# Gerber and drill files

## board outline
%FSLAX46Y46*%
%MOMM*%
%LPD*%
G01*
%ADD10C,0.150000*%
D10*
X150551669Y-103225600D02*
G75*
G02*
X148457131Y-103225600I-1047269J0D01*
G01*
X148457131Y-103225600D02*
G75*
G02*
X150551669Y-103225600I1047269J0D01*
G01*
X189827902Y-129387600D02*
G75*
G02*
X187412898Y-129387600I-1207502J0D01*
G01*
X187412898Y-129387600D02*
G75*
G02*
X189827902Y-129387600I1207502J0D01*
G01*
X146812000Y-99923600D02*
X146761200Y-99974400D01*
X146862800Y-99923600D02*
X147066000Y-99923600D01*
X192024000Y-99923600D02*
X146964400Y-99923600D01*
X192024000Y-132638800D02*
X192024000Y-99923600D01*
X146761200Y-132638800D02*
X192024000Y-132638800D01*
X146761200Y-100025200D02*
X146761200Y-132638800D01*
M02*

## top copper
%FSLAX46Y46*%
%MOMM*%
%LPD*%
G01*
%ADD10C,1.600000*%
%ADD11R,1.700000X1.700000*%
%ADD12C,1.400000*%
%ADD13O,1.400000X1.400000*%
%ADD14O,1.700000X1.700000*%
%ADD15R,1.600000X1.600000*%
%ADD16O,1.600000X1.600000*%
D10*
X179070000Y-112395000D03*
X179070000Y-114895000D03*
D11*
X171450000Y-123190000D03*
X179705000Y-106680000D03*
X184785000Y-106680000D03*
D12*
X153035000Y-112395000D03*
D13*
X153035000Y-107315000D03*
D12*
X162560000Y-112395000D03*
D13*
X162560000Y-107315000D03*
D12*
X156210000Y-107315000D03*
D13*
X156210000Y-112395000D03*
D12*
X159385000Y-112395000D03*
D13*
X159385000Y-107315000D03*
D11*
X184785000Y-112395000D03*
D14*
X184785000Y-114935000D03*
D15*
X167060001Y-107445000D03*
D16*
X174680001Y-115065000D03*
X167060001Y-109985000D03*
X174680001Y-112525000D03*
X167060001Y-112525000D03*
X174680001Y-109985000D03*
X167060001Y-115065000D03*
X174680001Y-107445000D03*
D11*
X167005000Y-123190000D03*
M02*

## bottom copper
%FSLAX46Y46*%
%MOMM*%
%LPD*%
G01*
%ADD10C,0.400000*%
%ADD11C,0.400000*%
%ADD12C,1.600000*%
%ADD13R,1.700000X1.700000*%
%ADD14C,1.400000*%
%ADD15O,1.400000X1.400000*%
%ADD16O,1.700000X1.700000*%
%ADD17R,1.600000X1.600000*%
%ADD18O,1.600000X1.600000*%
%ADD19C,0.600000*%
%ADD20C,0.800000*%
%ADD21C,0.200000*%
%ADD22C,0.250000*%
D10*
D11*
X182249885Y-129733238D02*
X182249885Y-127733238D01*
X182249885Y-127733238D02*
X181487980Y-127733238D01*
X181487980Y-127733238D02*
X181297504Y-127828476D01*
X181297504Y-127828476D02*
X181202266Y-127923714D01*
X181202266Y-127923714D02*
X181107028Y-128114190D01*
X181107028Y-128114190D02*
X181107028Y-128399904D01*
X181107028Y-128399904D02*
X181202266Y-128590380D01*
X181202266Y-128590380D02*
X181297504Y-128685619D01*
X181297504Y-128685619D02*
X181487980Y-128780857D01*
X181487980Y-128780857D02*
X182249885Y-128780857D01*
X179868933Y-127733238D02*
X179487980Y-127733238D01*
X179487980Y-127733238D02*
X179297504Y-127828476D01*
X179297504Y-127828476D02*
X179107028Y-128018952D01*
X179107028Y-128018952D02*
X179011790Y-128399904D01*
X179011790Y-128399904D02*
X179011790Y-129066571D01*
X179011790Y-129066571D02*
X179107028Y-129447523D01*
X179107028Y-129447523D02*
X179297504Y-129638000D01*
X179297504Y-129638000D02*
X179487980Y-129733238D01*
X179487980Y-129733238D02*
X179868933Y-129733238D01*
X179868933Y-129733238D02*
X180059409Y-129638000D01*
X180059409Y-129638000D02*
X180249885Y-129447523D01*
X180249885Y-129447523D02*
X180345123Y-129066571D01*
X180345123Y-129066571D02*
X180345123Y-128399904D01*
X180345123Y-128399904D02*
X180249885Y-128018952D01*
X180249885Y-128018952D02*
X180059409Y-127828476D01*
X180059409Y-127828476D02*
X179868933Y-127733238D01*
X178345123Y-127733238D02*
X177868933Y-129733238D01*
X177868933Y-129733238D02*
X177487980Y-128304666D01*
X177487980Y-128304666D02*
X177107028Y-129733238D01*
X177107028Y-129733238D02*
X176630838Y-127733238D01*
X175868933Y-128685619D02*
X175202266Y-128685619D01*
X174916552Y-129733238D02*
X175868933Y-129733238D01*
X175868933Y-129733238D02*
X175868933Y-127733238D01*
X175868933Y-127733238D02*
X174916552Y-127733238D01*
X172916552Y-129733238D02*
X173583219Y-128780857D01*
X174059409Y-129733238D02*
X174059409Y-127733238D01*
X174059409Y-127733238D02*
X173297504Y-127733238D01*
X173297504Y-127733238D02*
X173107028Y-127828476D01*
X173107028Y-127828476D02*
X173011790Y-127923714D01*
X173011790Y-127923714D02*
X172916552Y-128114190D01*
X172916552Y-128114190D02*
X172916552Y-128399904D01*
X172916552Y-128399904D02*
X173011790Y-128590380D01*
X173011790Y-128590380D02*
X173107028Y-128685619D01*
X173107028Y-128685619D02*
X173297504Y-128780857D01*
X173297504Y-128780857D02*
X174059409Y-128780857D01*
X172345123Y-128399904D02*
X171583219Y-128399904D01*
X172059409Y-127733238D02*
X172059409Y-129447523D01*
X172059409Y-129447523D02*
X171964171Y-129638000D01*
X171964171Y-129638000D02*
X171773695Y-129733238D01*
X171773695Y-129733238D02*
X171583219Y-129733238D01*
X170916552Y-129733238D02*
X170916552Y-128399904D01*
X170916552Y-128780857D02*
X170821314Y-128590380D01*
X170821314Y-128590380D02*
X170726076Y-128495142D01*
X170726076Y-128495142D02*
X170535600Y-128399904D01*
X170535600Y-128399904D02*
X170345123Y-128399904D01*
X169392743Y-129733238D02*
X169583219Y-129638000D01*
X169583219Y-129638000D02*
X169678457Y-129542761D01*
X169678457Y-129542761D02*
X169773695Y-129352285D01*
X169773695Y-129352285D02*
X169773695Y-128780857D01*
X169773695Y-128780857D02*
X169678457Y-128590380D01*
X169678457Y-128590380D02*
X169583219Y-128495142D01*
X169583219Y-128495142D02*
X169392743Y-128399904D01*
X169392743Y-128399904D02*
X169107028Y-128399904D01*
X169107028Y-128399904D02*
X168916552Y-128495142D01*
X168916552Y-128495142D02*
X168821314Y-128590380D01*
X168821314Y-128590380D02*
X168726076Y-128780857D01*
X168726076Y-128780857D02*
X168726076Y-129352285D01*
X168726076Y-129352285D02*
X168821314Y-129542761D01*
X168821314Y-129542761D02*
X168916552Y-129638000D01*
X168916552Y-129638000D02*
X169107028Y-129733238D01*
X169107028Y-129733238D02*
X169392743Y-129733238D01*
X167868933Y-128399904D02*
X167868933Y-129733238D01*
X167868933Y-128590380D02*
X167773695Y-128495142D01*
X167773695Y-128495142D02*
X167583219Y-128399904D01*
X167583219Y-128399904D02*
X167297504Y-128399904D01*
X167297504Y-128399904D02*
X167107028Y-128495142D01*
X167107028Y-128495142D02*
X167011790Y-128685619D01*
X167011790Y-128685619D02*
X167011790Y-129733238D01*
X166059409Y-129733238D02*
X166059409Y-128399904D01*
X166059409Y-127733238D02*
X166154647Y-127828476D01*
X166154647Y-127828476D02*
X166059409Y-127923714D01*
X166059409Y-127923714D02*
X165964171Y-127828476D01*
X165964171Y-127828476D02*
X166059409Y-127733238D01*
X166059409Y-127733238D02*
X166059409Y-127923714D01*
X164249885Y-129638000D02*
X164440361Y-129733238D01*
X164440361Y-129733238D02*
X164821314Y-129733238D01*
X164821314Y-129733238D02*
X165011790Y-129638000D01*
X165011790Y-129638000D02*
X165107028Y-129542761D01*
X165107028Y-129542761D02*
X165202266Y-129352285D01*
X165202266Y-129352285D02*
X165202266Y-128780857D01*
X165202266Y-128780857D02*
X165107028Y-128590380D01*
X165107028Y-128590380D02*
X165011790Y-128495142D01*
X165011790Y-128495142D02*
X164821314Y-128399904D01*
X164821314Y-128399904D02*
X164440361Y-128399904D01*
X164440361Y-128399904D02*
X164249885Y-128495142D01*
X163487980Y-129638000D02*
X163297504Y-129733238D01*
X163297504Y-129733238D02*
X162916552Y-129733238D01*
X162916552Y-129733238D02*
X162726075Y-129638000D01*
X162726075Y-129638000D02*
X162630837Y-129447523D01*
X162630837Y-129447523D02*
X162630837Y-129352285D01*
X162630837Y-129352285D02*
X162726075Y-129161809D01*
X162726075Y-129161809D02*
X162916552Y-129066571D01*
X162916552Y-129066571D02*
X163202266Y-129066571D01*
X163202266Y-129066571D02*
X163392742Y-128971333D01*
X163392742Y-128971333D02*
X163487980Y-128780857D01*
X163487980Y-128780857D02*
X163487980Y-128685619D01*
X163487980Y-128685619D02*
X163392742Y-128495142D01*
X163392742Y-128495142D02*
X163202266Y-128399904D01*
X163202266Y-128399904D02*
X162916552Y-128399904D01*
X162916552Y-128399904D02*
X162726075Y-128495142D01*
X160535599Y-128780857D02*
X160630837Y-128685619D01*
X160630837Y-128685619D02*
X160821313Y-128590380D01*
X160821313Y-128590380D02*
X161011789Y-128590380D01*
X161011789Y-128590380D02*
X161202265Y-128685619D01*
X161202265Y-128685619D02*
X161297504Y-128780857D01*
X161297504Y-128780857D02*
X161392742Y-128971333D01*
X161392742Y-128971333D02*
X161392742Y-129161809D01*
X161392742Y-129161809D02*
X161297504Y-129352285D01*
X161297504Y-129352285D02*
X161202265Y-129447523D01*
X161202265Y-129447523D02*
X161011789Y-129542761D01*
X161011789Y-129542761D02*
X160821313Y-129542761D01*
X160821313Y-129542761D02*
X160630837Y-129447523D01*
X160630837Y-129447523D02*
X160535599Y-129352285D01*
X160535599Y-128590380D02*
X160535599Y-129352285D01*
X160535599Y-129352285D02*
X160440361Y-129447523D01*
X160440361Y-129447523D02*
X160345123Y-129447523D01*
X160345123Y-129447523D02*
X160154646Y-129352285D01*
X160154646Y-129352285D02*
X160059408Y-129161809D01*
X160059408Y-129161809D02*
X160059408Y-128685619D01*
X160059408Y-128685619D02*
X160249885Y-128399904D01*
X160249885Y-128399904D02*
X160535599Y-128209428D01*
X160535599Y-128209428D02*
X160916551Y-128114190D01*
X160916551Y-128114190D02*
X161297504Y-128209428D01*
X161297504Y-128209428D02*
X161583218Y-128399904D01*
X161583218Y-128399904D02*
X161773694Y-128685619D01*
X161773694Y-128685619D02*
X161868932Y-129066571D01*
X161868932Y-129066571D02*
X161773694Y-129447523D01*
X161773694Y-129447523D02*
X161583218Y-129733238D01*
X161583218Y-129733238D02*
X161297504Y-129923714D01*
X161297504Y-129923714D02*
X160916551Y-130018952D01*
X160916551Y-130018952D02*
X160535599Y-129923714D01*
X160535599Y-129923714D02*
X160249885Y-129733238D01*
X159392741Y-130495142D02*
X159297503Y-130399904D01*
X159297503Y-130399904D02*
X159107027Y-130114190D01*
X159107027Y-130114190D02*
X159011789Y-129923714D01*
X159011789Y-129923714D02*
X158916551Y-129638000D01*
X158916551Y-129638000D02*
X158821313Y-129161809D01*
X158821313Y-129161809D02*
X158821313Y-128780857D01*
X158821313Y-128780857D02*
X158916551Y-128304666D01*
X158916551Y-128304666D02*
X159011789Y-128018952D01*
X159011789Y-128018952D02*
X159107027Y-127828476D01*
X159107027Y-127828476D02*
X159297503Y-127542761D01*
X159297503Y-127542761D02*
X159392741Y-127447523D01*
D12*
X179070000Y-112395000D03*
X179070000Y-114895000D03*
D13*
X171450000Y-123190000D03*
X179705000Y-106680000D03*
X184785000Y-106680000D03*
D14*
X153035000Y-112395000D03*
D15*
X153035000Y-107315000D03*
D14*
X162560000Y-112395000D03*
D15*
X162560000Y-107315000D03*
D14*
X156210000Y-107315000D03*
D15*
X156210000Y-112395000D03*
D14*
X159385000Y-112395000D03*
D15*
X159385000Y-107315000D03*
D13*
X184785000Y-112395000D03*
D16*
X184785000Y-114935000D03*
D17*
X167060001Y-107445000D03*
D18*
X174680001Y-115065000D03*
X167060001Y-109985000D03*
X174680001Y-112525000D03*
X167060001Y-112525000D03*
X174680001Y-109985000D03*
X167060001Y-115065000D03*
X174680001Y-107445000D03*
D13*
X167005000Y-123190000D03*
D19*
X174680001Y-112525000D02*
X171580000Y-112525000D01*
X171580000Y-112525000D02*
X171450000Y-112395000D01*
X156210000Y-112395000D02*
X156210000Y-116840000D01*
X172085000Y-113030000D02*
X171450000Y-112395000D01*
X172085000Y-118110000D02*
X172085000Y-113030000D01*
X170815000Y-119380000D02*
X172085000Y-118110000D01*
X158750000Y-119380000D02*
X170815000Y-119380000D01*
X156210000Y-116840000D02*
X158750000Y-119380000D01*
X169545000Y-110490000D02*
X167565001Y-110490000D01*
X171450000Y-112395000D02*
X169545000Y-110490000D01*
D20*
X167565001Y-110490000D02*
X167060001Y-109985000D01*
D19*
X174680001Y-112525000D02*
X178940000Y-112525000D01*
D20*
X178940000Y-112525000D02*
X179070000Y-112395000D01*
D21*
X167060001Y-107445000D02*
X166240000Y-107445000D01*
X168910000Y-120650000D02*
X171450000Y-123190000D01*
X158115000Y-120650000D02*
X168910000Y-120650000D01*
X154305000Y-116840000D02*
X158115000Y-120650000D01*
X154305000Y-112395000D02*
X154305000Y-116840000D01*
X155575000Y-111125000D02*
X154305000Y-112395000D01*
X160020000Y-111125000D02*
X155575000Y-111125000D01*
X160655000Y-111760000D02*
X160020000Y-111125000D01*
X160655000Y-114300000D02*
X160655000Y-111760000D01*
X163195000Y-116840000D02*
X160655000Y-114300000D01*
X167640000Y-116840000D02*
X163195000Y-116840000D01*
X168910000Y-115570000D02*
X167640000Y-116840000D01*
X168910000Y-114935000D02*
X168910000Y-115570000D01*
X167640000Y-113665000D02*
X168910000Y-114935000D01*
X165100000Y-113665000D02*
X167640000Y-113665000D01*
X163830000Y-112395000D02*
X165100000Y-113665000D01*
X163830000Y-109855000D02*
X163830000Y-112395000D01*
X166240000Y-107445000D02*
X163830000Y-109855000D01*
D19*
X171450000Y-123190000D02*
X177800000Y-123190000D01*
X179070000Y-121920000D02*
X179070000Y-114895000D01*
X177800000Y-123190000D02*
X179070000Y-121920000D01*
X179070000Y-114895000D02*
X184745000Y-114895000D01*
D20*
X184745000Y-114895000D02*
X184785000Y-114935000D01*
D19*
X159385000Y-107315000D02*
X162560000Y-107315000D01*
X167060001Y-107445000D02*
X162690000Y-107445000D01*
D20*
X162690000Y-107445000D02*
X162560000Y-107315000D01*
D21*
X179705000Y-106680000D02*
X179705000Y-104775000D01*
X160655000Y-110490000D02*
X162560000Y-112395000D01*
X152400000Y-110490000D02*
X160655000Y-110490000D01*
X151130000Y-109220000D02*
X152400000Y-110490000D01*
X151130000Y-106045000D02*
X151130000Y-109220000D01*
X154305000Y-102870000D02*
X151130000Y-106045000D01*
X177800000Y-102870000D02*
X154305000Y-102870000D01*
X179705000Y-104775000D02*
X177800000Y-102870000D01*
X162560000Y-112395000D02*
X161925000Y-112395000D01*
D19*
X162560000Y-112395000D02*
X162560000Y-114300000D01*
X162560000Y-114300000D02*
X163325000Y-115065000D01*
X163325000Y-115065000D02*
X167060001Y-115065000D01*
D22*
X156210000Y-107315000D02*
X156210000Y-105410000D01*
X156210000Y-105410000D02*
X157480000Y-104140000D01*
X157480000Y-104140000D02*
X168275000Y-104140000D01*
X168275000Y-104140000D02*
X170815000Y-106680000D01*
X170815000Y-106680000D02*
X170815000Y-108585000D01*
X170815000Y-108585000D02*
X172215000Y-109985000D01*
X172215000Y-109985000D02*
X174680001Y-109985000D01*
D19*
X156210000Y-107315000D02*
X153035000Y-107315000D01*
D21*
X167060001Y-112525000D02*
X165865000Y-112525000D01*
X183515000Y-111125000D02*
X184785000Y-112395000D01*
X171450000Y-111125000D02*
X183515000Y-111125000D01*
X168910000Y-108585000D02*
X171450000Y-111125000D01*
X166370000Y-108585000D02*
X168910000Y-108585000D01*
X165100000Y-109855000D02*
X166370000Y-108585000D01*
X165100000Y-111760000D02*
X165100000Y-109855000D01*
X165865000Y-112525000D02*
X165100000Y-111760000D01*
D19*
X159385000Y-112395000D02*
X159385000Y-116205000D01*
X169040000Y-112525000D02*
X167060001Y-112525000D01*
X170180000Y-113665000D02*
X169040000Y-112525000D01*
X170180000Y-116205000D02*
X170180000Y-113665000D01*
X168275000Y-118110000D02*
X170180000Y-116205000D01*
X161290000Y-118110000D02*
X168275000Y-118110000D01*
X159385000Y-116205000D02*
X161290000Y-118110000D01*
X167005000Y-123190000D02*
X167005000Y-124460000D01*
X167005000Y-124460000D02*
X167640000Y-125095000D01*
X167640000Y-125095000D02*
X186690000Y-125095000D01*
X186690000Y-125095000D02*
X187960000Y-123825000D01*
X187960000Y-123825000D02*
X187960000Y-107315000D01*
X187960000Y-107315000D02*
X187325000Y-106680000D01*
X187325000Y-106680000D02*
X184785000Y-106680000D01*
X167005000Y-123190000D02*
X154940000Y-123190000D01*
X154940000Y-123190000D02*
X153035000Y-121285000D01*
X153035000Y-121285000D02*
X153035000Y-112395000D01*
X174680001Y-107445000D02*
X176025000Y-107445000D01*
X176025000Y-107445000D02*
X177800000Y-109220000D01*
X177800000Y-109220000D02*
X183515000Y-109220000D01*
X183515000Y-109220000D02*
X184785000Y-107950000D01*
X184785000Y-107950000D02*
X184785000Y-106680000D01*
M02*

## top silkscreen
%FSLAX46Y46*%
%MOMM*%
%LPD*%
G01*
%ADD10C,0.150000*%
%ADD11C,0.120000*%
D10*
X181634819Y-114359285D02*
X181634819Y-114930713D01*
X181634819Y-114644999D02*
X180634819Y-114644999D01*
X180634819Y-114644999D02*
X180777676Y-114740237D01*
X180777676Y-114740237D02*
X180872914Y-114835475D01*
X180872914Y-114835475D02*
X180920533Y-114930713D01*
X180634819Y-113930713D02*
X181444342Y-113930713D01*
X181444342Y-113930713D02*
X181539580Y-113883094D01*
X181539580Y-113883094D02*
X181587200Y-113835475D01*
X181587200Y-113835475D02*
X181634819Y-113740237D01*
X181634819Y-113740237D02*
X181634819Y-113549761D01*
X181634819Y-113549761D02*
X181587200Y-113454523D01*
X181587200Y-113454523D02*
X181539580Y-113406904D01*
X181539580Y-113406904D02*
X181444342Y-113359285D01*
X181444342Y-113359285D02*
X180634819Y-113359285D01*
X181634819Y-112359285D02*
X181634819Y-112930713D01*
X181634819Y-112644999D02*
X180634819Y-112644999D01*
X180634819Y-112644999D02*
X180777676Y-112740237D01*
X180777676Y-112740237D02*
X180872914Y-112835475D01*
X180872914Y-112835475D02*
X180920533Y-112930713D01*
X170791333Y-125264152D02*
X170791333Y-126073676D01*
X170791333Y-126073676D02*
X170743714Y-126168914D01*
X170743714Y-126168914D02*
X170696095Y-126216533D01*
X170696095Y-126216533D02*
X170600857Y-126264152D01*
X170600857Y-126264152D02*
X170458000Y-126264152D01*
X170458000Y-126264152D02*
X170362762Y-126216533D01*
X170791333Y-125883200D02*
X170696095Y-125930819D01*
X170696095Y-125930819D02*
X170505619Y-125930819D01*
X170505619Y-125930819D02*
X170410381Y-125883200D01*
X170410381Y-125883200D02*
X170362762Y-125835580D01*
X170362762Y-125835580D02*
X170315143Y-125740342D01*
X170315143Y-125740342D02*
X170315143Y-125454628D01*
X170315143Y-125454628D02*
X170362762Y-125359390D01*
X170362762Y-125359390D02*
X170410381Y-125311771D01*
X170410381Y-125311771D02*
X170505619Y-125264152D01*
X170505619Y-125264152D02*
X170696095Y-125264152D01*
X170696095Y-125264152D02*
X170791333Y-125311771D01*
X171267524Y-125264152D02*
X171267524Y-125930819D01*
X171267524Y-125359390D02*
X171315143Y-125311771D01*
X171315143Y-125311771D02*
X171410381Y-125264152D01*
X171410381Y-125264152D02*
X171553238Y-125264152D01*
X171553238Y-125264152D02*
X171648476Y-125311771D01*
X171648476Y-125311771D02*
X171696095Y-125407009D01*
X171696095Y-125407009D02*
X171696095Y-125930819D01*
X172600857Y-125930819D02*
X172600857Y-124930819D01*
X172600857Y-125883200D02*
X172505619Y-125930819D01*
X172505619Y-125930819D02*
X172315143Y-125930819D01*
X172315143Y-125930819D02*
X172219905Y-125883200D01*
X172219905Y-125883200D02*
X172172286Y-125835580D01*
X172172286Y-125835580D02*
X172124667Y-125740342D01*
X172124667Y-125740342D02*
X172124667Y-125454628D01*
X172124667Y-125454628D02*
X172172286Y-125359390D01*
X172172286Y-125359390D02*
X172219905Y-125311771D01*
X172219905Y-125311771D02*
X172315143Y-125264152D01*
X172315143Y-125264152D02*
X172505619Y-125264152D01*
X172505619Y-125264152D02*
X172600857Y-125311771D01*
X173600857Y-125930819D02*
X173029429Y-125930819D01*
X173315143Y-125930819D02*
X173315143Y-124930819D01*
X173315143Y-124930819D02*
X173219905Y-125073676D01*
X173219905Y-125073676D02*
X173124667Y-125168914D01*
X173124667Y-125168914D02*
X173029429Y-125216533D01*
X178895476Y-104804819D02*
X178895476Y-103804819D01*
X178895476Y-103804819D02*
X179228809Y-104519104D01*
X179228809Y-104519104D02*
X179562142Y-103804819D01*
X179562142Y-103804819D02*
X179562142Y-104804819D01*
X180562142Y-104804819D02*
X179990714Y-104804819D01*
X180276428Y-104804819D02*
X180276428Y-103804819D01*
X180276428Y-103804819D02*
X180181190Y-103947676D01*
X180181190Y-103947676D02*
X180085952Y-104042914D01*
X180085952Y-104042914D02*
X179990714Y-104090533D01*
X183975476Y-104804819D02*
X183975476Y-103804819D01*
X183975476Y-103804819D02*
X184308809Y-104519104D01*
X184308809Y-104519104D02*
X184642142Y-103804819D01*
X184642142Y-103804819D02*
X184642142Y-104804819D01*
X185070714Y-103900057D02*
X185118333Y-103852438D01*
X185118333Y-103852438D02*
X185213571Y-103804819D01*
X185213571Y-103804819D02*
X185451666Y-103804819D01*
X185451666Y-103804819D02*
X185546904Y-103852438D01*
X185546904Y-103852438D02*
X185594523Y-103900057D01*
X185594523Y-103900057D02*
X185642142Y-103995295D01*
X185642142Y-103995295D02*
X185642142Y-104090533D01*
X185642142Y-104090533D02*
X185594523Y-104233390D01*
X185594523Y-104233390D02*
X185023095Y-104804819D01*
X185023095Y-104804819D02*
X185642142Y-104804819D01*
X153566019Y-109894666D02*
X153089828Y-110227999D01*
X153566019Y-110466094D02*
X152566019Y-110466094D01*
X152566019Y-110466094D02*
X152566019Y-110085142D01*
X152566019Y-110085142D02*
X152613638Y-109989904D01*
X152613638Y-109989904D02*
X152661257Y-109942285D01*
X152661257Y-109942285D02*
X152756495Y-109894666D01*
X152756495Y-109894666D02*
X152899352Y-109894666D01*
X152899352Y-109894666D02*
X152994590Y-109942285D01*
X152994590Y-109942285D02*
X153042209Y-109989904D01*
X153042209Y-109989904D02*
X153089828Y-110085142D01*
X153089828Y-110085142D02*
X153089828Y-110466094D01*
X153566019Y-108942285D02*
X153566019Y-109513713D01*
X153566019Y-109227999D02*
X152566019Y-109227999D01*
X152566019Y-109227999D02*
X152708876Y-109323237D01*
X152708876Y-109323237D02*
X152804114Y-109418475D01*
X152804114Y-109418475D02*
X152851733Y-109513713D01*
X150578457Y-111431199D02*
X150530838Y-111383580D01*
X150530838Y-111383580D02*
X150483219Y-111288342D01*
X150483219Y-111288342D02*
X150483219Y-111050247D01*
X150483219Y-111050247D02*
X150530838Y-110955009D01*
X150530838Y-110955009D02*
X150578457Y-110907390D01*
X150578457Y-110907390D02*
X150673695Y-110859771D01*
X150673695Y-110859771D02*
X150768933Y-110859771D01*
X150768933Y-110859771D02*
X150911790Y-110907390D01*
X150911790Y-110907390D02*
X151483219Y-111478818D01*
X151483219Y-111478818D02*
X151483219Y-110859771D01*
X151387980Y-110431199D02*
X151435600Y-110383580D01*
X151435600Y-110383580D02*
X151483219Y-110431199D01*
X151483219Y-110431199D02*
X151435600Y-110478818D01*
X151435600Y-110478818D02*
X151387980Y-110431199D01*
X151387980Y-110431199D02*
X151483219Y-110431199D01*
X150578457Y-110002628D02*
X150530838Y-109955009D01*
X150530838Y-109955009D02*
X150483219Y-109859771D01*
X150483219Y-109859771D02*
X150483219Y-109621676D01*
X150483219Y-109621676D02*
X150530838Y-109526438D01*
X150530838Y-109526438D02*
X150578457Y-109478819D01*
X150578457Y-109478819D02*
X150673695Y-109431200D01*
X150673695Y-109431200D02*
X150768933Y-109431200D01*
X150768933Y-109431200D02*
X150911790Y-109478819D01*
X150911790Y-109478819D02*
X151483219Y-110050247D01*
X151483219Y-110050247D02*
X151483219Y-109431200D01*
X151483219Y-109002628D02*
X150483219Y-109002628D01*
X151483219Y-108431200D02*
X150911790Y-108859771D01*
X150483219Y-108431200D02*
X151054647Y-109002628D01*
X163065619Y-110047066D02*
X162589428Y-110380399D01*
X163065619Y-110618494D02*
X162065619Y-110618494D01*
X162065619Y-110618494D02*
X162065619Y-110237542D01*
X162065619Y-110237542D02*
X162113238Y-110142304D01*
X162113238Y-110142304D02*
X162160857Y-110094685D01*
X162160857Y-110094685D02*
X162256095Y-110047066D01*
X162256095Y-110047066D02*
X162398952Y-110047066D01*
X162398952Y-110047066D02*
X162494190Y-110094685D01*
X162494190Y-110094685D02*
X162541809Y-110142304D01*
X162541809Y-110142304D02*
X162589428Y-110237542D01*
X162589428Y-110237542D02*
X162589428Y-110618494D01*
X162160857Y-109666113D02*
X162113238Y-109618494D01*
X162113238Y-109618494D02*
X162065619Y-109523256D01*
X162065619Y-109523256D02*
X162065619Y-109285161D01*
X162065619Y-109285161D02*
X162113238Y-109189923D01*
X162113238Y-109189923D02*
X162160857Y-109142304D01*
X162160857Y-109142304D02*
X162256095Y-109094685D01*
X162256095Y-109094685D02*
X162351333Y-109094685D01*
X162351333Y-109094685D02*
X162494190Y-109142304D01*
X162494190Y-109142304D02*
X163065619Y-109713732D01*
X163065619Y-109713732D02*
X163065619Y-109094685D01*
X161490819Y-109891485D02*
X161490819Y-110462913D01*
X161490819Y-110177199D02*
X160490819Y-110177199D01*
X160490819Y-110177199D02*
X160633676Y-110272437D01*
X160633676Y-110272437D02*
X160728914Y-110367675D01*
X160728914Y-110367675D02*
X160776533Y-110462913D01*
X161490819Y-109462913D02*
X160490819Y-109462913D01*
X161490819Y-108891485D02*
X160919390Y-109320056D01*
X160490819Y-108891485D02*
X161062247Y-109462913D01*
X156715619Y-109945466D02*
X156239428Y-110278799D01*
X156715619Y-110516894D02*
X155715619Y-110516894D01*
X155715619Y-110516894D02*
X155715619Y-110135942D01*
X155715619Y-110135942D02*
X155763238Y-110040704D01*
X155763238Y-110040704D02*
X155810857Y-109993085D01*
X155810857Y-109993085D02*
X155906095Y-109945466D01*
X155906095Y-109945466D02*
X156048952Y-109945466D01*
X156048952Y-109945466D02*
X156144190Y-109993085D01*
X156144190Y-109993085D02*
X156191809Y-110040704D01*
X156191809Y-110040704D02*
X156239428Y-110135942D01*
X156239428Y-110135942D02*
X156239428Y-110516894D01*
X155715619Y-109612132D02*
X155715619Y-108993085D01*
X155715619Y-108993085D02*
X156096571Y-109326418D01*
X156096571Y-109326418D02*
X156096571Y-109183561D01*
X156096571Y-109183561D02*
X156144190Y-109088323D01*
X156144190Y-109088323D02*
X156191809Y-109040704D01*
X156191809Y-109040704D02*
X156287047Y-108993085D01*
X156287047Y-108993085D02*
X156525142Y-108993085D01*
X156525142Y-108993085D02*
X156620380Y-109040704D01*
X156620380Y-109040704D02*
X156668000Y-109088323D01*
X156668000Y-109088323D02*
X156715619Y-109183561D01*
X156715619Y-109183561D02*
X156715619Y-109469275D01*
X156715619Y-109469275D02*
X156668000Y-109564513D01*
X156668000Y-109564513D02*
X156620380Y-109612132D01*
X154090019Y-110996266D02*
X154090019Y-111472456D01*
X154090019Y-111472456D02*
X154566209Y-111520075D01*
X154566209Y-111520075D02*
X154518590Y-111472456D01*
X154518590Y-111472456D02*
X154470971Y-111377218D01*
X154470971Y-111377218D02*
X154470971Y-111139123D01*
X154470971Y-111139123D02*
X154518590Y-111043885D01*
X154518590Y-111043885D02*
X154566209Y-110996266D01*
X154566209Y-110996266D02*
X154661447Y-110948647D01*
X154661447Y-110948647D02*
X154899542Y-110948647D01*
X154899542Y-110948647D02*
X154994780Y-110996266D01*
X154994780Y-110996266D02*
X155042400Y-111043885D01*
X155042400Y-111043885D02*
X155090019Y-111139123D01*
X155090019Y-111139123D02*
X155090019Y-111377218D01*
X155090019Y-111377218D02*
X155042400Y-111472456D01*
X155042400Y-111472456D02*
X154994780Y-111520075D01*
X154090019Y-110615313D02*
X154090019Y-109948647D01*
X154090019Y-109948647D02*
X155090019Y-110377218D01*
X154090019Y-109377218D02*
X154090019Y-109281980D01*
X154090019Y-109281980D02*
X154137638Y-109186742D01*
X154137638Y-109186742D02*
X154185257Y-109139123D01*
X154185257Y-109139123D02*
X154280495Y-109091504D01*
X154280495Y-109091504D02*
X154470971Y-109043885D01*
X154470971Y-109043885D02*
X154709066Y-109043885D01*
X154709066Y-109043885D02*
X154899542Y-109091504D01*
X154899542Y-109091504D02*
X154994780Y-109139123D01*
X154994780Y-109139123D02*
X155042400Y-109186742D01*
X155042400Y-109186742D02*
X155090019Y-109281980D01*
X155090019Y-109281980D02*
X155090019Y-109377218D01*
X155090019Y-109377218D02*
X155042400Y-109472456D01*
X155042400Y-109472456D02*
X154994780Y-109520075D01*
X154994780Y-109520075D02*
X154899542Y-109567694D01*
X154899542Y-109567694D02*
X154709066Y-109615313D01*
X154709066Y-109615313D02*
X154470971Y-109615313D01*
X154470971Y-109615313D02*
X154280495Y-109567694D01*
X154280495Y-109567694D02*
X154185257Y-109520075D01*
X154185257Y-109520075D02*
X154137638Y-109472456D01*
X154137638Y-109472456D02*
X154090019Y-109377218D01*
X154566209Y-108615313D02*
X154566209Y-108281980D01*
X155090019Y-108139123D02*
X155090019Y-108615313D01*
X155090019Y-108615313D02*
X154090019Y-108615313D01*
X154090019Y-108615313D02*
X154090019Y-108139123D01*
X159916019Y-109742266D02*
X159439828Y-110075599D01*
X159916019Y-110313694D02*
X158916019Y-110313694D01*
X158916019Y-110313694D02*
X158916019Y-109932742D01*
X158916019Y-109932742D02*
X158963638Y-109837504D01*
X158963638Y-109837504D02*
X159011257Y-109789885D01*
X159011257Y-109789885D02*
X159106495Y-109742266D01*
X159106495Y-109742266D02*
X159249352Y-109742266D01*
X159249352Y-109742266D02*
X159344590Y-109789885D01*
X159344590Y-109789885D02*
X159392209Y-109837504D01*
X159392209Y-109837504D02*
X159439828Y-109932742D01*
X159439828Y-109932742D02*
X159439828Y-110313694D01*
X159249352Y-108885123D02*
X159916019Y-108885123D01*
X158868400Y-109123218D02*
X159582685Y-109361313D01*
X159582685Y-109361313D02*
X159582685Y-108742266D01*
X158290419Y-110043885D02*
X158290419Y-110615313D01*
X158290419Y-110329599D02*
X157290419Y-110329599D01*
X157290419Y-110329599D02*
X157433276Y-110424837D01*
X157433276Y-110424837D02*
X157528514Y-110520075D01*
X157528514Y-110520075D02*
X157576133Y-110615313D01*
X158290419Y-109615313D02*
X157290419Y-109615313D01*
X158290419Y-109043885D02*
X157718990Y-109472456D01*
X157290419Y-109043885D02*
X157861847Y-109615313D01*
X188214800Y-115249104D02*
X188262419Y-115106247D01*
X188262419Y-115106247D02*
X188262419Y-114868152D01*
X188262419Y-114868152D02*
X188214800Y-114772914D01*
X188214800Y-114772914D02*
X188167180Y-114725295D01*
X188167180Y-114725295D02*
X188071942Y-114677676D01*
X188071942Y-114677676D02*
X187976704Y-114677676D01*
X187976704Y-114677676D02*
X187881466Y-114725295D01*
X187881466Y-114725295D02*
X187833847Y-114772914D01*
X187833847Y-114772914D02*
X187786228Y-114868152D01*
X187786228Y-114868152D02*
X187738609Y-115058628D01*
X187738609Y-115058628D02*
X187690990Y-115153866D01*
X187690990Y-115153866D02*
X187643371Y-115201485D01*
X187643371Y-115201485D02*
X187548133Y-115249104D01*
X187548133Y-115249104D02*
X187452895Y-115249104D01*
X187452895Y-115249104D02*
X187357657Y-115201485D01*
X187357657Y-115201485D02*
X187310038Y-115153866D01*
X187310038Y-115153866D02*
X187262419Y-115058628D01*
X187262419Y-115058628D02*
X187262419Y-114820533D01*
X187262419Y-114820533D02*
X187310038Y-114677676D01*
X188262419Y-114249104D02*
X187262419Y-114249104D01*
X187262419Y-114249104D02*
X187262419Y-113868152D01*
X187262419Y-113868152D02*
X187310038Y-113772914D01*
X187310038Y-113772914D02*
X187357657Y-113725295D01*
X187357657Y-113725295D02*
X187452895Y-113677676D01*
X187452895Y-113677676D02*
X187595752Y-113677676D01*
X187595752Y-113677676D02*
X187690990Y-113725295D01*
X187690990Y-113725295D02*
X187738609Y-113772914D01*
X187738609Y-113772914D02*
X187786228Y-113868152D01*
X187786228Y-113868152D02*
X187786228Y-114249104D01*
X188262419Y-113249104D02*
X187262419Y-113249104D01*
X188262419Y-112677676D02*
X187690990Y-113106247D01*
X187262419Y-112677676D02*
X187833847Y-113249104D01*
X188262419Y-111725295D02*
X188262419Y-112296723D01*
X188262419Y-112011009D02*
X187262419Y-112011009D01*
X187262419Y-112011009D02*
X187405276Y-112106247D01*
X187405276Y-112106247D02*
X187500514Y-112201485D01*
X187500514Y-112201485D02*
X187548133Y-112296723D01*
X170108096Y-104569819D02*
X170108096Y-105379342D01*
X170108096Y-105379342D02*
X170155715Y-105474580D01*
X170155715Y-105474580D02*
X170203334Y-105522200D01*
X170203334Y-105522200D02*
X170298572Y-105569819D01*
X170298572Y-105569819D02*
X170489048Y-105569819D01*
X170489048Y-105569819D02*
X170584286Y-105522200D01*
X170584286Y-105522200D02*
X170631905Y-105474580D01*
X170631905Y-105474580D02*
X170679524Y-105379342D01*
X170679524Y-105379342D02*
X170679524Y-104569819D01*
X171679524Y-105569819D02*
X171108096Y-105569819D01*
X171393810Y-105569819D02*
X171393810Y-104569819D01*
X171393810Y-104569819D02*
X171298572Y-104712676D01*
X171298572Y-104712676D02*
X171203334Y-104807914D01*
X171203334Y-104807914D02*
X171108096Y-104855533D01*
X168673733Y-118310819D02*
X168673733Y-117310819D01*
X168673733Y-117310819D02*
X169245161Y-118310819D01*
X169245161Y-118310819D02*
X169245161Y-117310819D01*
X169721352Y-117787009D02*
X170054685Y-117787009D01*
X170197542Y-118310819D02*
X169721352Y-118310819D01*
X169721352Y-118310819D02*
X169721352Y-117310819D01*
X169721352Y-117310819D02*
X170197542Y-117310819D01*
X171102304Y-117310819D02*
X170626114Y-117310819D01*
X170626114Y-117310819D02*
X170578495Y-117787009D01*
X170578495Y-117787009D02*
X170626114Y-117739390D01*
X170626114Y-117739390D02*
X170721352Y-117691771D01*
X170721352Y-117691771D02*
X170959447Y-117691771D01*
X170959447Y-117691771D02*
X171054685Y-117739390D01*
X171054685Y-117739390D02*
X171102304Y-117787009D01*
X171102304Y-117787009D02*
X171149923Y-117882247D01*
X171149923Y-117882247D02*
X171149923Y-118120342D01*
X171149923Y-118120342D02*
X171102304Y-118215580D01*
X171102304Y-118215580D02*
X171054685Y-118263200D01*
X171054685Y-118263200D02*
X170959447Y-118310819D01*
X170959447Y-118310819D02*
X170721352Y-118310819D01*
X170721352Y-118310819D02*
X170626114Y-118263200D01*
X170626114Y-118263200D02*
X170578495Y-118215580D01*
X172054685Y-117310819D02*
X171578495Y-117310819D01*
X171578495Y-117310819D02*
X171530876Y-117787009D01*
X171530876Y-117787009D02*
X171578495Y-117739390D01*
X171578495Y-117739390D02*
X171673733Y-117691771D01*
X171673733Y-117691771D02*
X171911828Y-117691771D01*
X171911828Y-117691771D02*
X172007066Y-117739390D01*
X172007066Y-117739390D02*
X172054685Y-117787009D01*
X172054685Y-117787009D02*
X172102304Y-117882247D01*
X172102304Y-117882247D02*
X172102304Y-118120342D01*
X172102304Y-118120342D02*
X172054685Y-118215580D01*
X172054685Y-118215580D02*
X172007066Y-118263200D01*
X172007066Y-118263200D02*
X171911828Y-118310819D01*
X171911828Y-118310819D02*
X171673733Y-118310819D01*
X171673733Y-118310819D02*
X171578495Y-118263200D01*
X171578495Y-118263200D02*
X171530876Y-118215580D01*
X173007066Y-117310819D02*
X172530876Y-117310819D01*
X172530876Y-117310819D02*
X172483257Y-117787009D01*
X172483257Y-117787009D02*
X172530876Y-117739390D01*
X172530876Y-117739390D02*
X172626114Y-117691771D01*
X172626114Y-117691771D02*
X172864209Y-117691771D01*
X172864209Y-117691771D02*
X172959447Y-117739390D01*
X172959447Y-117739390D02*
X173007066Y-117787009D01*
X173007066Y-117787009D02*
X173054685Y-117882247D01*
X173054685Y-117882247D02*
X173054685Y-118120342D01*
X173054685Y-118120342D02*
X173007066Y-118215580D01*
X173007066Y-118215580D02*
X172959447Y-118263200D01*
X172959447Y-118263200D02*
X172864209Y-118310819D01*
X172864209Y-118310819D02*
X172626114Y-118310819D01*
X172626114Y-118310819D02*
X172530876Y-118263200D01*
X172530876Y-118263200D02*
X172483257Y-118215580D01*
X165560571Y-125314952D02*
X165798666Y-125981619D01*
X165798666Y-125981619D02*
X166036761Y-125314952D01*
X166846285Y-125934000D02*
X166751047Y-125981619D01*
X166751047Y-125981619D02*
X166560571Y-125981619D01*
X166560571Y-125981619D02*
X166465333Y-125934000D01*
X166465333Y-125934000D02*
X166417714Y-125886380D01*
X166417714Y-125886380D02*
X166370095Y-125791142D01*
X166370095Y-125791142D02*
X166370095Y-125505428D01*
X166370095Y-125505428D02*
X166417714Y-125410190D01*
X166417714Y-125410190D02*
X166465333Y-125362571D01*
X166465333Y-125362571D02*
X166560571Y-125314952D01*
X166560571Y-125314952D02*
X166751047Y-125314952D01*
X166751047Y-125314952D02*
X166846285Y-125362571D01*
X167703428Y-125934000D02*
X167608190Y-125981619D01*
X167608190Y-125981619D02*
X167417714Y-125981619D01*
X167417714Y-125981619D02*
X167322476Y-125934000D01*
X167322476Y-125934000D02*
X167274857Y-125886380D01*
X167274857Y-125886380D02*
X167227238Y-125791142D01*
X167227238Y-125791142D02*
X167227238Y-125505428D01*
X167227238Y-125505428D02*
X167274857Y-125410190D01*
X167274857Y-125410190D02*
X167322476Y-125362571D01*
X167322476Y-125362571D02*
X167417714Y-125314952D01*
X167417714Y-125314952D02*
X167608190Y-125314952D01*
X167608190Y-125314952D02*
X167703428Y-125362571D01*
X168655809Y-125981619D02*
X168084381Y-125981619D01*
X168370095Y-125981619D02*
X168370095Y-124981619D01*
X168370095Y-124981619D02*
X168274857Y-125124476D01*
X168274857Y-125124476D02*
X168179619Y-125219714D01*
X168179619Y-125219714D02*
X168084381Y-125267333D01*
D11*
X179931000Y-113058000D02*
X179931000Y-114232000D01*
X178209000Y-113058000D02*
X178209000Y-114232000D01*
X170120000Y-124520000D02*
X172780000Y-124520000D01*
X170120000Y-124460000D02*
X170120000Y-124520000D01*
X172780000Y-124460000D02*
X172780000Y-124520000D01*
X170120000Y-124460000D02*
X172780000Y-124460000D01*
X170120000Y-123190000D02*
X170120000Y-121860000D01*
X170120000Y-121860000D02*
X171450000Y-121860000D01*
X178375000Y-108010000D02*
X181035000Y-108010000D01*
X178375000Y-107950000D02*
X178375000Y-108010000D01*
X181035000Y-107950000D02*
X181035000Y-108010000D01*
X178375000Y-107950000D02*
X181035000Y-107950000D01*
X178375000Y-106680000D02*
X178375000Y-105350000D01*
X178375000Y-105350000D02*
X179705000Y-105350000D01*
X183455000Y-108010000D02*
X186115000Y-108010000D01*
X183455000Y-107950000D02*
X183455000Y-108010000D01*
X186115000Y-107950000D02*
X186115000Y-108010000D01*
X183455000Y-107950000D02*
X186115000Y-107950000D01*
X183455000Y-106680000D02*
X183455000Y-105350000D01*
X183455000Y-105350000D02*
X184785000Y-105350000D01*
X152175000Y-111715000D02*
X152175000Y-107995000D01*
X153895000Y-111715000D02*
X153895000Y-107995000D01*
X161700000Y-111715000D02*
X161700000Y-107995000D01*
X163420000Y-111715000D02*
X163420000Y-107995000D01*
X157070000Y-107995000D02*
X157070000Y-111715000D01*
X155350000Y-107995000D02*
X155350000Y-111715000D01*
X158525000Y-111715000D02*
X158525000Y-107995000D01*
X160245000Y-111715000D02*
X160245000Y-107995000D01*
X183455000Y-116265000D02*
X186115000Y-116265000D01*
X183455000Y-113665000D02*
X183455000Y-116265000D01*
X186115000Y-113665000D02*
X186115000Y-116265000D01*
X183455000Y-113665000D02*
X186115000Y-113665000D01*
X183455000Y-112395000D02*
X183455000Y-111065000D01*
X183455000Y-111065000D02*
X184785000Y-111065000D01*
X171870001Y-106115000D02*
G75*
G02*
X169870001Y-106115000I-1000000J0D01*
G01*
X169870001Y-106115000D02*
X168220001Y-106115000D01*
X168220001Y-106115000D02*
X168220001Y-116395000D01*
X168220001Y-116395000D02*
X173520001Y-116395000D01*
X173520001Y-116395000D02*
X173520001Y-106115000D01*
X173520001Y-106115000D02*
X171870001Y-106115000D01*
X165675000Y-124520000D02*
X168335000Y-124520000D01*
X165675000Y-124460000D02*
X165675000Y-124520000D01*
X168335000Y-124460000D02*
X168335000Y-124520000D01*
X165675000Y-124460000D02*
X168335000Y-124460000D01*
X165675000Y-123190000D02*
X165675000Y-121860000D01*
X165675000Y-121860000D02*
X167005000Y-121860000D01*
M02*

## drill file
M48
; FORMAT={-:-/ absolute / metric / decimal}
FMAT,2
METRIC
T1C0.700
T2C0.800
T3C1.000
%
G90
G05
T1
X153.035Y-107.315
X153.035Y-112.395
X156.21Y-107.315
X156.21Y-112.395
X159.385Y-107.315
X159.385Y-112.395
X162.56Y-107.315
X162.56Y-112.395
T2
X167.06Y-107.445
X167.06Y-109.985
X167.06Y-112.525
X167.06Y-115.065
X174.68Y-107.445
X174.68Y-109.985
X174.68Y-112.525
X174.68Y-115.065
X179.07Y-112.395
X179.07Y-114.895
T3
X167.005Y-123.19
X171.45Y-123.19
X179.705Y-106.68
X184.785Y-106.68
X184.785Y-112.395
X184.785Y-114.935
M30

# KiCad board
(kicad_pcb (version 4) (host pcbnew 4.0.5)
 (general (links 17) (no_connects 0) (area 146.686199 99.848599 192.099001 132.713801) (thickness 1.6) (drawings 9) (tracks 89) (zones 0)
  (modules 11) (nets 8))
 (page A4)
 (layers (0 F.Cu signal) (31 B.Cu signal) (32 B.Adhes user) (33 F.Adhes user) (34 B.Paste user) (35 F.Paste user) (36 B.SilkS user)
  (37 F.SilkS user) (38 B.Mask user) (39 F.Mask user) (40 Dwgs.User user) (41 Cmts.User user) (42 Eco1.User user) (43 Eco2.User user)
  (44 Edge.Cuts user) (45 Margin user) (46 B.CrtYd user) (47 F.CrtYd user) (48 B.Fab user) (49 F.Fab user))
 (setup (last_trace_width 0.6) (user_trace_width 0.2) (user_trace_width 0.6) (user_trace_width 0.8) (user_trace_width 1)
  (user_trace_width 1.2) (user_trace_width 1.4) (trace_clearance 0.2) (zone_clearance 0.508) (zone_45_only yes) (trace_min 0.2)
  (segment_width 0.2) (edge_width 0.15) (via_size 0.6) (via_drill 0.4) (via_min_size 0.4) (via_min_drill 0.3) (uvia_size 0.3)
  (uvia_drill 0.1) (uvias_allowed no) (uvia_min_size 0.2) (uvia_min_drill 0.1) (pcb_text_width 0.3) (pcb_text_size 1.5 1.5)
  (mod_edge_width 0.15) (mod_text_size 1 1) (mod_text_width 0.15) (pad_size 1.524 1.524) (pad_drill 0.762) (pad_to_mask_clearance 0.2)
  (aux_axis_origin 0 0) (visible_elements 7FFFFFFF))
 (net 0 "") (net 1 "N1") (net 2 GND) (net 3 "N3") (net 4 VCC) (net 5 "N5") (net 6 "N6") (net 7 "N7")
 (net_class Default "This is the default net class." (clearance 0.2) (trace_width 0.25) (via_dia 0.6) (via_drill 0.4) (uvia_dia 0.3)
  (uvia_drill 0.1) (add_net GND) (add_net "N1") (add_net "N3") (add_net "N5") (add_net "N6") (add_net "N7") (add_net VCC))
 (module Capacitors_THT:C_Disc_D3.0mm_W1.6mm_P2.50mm (layer F.Cu) (at 179.07 112.395 270)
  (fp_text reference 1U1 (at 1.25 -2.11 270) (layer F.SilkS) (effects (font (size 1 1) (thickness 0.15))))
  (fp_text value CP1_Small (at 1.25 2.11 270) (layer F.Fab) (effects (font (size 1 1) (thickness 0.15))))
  (fp_line (start 0.663 -0.861) (end 1.837 -0.861) (layer F.SilkS) (width 0.12))
  (fp_line (start 0.663 0.861) (end 1.837 0.861) (layer F.SilkS) (width 0.12))
  (pad 1 thru_hole circle (at 0 0 270) (size 1.6 1.6) (drill 0.8) (layers *.Cu *.Mask) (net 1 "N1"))
  (pad 2 thru_hole circle (at 2.5 0 270) (size 1.6 1.6) (drill 0.8) (layers *.Cu *.Mask) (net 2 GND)))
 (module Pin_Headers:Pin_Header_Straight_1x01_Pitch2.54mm (layer F.Cu) (at 171.45 123.19)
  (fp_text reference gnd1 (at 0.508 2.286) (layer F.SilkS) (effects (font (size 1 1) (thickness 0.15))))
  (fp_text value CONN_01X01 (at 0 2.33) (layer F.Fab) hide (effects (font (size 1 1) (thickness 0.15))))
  (fp_line (start -1.33 1.33) (end 1.33 1.33) (layer F.SilkS) (width 0.12))
  (fp_line (start -1.33 1.27) (end -1.33 1.33) (layer F.SilkS) (width 0.12))
  (fp_line (start 1.33 1.27) (end 1.33 1.33) (layer F.SilkS) (width 0.12))
  (fp_line (start -1.33 1.27) (end 1.33 1.27) (layer F.SilkS) (width 0.12))
  (fp_line (start -1.33 0) (end -1.33 -1.33) (layer F.SilkS) (width 0.12))
  (fp_line (start -1.33 -1.33) (end 0 -1.33) (layer F.SilkS) (width 0.12))
  (pad 1 thru_hole rect (at 0 0) (size 1.7 1.7) (drill 1) (layers *.Cu *.Mask) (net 2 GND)))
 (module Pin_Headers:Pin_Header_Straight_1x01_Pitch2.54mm (layer F.Cu) (at 179.705 106.68)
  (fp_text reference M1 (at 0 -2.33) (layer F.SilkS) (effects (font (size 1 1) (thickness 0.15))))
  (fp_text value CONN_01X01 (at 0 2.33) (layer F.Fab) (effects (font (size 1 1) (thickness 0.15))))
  (fp_line (start -1.33 1.33) (end 1.33 1.33) (layer F.SilkS) (width 0.12))
  (fp_line (start -1.33 1.27) (end -1.33 1.33) (layer F.SilkS) (width 0.12))
  (fp_line (start 1.33 1.27) (end 1.33 1.33) (layer F.SilkS) (width 0.12))
  (fp_line (start -1.33 1.27) (end 1.33 1.27) (layer F.SilkS) (width 0.12))
  (fp_line (start -1.33 0) (end -1.33 -1.33) (layer F.SilkS) (width 0.12))
  (fp_line (start -1.33 -1.33) (end 0 -1.33) (layer F.SilkS) (width 0.12))
  (pad 1 thru_hole rect (at 0 0) (size 1.7 1.7) (drill 1) (layers *.Cu *.Mask) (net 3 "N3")))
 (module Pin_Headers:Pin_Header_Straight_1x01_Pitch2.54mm (layer F.Cu) (at 184.785 106.68)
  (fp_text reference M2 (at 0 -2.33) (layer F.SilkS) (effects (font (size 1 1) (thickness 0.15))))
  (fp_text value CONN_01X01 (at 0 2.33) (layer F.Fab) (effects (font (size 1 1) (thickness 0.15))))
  (fp_line (start -1.33 1.33) (end 1.33 1.33) (layer F.SilkS) (width 0.12))
  (fp_line (start -1.33 1.27) (end -1.33 1.33) (layer F.SilkS) (width 0.12))
  (fp_line (start 1.33 1.27) (end 1.33 1.33) (layer F.SilkS) (width 0.12))
  (fp_line (start -1.33 1.27) (end 1.33 1.27) (layer F.SilkS) (width 0.12))
  (fp_line (start -1.33 0) (end -1.33 -1.33) (layer F.SilkS) (width 0.12))
  (fp_line (start -1.33 -1.33) (end 0 -1.33) (layer F.SilkS) (width 0.12))
  (pad 1 thru_hole rect (at 0 0) (size 1.7 1.7) (drill 1) (layers *.Cu *.Mask) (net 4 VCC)))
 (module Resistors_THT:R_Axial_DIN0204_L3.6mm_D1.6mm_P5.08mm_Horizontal (layer F.Cu) (at 153.035 112.395 90)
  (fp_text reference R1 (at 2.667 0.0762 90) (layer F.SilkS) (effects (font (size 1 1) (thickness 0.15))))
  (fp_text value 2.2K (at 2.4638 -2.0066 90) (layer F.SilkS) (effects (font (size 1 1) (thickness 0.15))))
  (fp_line (start 0.68 -0.86) (end 4.4 -0.86) (layer F.SilkS) (width 0.12))
  (fp_line (start 0.68 0.86) (end 4.4 0.86) (layer F.SilkS) (width 0.12))
  (pad 1 thru_hole circle (at 0 0 90) (size 1.4 1.4) (drill 0.7) (layers *.Cu *.Mask) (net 4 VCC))
  (pad 2 thru_hole oval (at 5.08 0 90) (size 1.4 1.4) (drill 0.7) (layers *.Cu *.Mask) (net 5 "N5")))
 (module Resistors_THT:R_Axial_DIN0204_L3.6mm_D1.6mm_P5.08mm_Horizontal (layer F.Cu) (at 162.56 112.395 90)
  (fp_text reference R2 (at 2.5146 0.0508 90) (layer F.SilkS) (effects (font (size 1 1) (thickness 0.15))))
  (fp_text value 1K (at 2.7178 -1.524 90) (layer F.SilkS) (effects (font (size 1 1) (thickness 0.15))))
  (fp_line (start 0.68 -0.86) (end 4.4 -0.86) (layer F.SilkS) (width 0.12))
  (fp_line (start 0.68 0.86) (end 4.4 0.86) (layer F.SilkS) (width 0.12))
  (pad 1 thru_hole circle (at 0 0 90) (size 1.4 1.4) (drill 0.7) (layers *.Cu *.Mask) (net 3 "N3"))
  (pad 2 thru_hole oval (at 5.08 0 90) (size 1.4 1.4) (drill 0.7) (layers *.Cu *.Mask) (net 2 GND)))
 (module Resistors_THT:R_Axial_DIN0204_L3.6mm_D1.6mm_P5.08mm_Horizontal (layer F.Cu) (at 156.21 107.315 270)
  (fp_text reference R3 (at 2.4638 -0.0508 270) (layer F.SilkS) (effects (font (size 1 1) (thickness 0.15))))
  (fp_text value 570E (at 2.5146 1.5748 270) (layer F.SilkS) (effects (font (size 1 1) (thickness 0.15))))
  (fp_line (start 0.68 -0.86) (end 4.4 -0.86) (layer F.SilkS) (width 0.12))
  (fp_line (start 0.68 0.86) (end 4.4 0.86) (layer F.SilkS) (width 0.12))
  (pad 1 thru_hole circle (at 0 0 270) (size 1.4 1.4) (drill 0.7) (layers *.Cu *.Mask) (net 5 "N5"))
  (pad 2 thru_hole oval (at 5.08 0 270) (size 1.4 1.4) (drill 0.7) (layers *.Cu *.Mask) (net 1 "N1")))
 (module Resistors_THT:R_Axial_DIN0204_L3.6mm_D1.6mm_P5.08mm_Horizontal (layer F.Cu) (at 159.385 112.395 90)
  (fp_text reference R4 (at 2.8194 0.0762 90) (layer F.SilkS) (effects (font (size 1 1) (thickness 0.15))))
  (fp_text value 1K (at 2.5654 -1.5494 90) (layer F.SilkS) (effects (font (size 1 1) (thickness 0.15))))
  (fp_line (start 0.68 -0.86) (end 4.4 -0.86) (layer F.SilkS) (width 0.12))
  (fp_line (start 0.68 0.86) (end 4.4 0.86) (layer F.SilkS) (width 0.12))
  (pad 1 thru_hole circle (at 0 0 90) (size 1.4 1.4) (drill 0.7) (layers *.Cu *.Mask) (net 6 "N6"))
  (pad 2 thru_hole oval (at 5.08 0 90) (size 1.4 1.4) (drill 0.7) (layers *.Cu *.Mask) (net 2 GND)))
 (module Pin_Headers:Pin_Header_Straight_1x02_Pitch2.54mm (layer F.Cu) (at 184.785 112.395)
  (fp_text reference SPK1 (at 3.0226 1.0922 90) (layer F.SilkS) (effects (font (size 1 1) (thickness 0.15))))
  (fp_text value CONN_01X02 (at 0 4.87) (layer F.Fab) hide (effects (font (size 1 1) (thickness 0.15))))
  (fp_line (start -1.33 3.87) (end 1.33 3.87) (layer F.SilkS) (width 0.12))
  (fp_line (start -1.33 1.27) (end -1.33 3.87) (layer F.SilkS) (width 0.12))
  (fp_line (start 1.33 1.27) (end 1.33 3.87) (layer F.SilkS) (width 0.12))
  (fp_line (start -1.33 1.27) (end 1.33 1.27) (layer F.SilkS) (width 0.12))
  (fp_line (start -1.33 0) (end -1.33 -1.33) (layer F.SilkS) (width 0.12))
  (fp_line (start -1.33 -1.33) (end 0 -1.33) (layer F.SilkS) (width 0.12))
  (pad 1 thru_hole rect (at 0 0) (size 1.7 1.7) (drill 1) (layers *.Cu *.Mask) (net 6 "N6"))
  (pad 2 thru_hole oval (at 0 2.54) (size 1.7 1.7) (drill 1) (layers *.Cu *.Mask) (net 2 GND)))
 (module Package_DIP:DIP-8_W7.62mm (layer F.Cu) (at 167.060001 107.445)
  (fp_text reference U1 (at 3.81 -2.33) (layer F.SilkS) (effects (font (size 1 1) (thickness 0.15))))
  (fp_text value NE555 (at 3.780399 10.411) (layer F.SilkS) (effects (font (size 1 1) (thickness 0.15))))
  (fp_arc (start 3.81 -1.33) (end 2.81 -1.33) (angle -180) (layer F.SilkS) (width 0.12))
  (fp_line (start 2.81 -1.33) (end 1.16 -1.33) (layer F.SilkS) (width 0.12))
  (fp_line (start 1.16 -1.33) (end 1.16 8.95) (layer F.SilkS) (width 0.12))
  (fp_line (start 1.16 8.95) (end 6.46 8.95) (layer F.SilkS) (width 0.12))
  (fp_line (start 6.46 8.95) (end 6.46 -1.33) (layer F.SilkS) (width 0.12))
  (fp_line (start 6.46 -1.33) (end 4.81 -1.33) (layer F.SilkS) (width 0.12))
  (pad 1 thru_hole rect (at 0 0) (size 1.6 1.6) (drill 0.8) (layers *.Cu *.Mask) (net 2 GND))
  (pad 5 thru_hole oval (at 7.62 7.62) (size 1.6 1.6) (drill 0.8) (layers *.Cu *.Mask) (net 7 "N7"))
  (pad 2 thru_hole oval (at 0 2.54) (size 1.6 1.6) (drill 0.8) (layers *.Cu *.Mask) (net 1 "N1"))
  (pad 6 thru_hole oval (at 7.62 5.08) (size 1.6 1.6) (drill 0.8) (layers *.Cu *.Mask) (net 1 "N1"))
  (pad 3 thru_hole oval (at 0 5.08) (size 1.6 1.6) (drill 0.8) (layers *.Cu *.Mask) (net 6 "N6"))
  (pad 7 thru_hole oval (at 7.62 2.54) (size 1.6 1.6) (drill 0.8) (layers *.Cu *.Mask) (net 5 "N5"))
  (pad 4 thru_hole oval (at 0 7.62) (size 1.6 1.6) (drill 0.8) (layers *.Cu *.Mask) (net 3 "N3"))
  (pad 8 thru_hole oval (at 7.62 0) (size 1.6 1.6) (drill 0.8) (layers *.Cu *.Mask) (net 4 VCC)))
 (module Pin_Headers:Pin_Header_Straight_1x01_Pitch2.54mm (layer F.Cu) (at 167.005 123.19)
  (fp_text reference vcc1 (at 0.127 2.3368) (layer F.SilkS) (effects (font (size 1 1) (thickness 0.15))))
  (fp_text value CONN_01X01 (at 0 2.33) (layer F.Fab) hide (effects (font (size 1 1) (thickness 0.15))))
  (fp_line (start -1.33 1.33) (end 1.33 1.33) (layer F.SilkS) (width 0.12))
  (fp_line (start -1.33 1.27) (end -1.33 1.33) (layer F.SilkS) (width 0.12))
  (fp_line (start 1.33 1.27) (end 1.33 1.33) (layer F.SilkS) (width 0.12))
  (fp_line (start -1.33 1.27) (end 1.33 1.27) (layer F.SilkS) (width 0.12))
  (fp_line (start -1.33 0) (end -1.33 -1.33) (layer F.SilkS) (width 0.12))
  (fp_line (start -1.33 -1.33) (end 0 -1.33) (layer F.SilkS) (width 0.12))
  (pad 1 thru_hole rect (at 0 0) (size 1.7 1.7) (drill 1) (layers *.Cu *.Mask) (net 4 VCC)))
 (gr_circle (center 149.5044 103.2256) (end 149.098 102.2604) (layer Edge.Cuts) (width 0.15))
 (gr_circle (center 188.6204 129.3876) (end 188.1632 128.27) (layer Edge.Cuts) (width 0.15))
 (gr_line (start 146.812 99.9236) (end 146.7612 99.9744) (angle 90) (layer Edge.Cuts) (width 0.15))
 (gr_line (start 146.8628 99.9236) (end 147.066 99.9236) (angle 90) (layer Edge.Cuts) (width 0.15))
 (gr_line (start 192.024 99.9236) (end 146.9644 99.9236) (angle 90) (layer Edge.Cuts) (width 0.15))
 (gr_line (start 192.024 132.6388) (end 192.024 99.9236) (angle 90) (layer Edge.Cuts) (width 0.15))
 (gr_line (start 146.7612 132.6388) (end 192.024 132.6388) (angle 90) (layer Edge.Cuts) (width 0.15))
 (gr_line (start 146.7612 100.0252) (end 146.7612 132.6388) (angle 90) (layer Edge.Cuts) (width 0.15))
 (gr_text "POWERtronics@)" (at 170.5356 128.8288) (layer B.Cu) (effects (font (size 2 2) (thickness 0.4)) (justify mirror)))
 (segment (start 174.680001 112.525) (end 171.58 112.525) (width 0.6) (layer B.Cu) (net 1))
 (segment (start 171.58 112.525) (end 171.45 112.395) (width 0.6) (layer B.Cu) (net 1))
 (segment (start 156.21 112.395) (end 156.21 116.84) (width 0.6) (layer B.Cu) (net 1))
 (segment (start 172.085 113.03) (end 171.45 112.395) (width 0.6) (layer B.Cu) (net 1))
 (segment (start 172.085 118.11) (end 172.085 113.03) (width 0.6) (layer B.Cu) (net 1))
 (segment (start 170.815 119.38) (end 172.085 118.11) (width 0.6) (layer B.Cu) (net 1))
 (segment (start 158.75 119.38) (end 170.815 119.38) (width 0.6) (layer B.Cu) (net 1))
 (segment (start 156.21 116.84) (end 158.75 119.38) (width 0.6) (layer B.Cu) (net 1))
 (segment (start 169.545 110.49) (end 167.565001 110.49) (width 0.6) (layer B.Cu) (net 1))
 (segment (start 171.45 112.395) (end 169.545 110.49) (width 0.6) (layer B.Cu) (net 1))
 (segment (start 167.565001 110.49) (end 167.060001 109.985) (width 0.8) (layer B.Cu) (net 1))
 (segment (start 174.680001 112.525) (end 178.94 112.525) (width 0.6) (layer B.Cu) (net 1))
 (segment (start 178.94 112.525) (end 179.07 112.395) (width 0.8) (layer B.Cu) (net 1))
 (segment (start 167.060001 107.445) (end 166.24 107.445) (width 0.2) (layer B.Cu) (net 2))
 (segment (start 168.91 120.65) (end 171.45 123.19) (width 0.2) (layer B.Cu) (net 2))
 (segment (start 158.115 120.65) (end 168.91 120.65) (width 0.2) (layer B.Cu) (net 2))
 (segment (start 154.305 116.84) (end 158.115 120.65) (width 0.2) (layer B.Cu) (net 2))
 (segment (start 154.305 112.395) (end 154.305 116.84) (width 0.2) (layer B.Cu) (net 2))
 (segment (start 155.575 111.125) (end 154.305 112.395) (width 0.2) (layer B.Cu) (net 2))
 (segment (start 160.02 111.125) (end 155.575 111.125) (width 0.2) (layer B.Cu) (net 2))
 (segment (start 160.655 111.76) (end 160.02 111.125) (width 0.2) (layer B.Cu) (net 2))
 (segment (start 160.655 114.3) (end 160.655 111.76) (width 0.2) (layer B.Cu) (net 2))
 (segment (start 163.195 116.84) (end 160.655 114.3) (width 0.2) (layer B.Cu) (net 2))
 (segment (start 167.64 116.84) (end 163.195 116.84) (width 0.2) (layer B.Cu) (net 2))
 (segment (start 168.91 115.57) (end 167.64 116.84) (width 0.2) (layer B.Cu) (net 2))
 (segment (start 168.91 114.935) (end 168.91 115.57) (width 0.2) (layer B.Cu) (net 2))
 (segment (start 167.64 113.665) (end 168.91 114.935) (width 0.2) (layer B.Cu) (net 2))
 (segment (start 165.1 113.665) (end 167.64 113.665) (width 0.2) (layer B.Cu) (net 2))
 (segment (start 163.83 112.395) (end 165.1 113.665) (width 0.2) (layer B.Cu) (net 2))
 (segment (start 163.83 109.855) (end 163.83 112.395) (width 0.2) (layer B.Cu) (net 2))
 (segment (start 166.24 107.445) (end 163.83 109.855) (width 0.2) (layer B.Cu) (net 2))
 (segment (start 171.45 123.19) (end 177.8 123.19) (width 0.6) (layer B.Cu) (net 2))
 (segment (start 179.07 121.92) (end 179.07 114.895) (width 0.6) (layer B.Cu) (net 2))
 (segment (start 177.8 123.19) (end 179.07 121.92) (width 0.6) (layer B.Cu) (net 2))
 (segment (start 179.07 114.895) (end 184.745 114.895) (width 0.6) (layer B.Cu) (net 2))
 (segment (start 184.745 114.895) (end 184.785 114.935) (width 0.8) (layer B.Cu) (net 2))
 (segment (start 159.385 107.315) (end 162.56 107.315) (width 0.6) (layer B.Cu) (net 2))
 (segment (start 167.060001 107.445) (end 162.69 107.445) (width 0.6) (layer B.Cu) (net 2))
 (segment (start 162.69 107.445) (end 162.56 107.315) (width 0.8) (layer B.Cu) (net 2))
 (segment (start 179.705 106.68) (end 179.705 104.775) (width 0.2) (layer B.Cu) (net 3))
 (segment (start 160.655 110.49) (end 162.56 112.395) (width 0.2) (layer B.Cu) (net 3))
 (segment (start 152.4 110.49) (end 160.655 110.49) (width 0.2) (layer B.Cu) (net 3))
 (segment (start 151.13 109.22) (end 152.4 110.49) (width 0.2) (layer B.Cu) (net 3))
 (segment (start 151.13 106.045) (end 151.13 109.22) (width 0.2) (layer B.Cu) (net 3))
 (segment (start 154.305 102.87) (end 151.13 106.045) (width 0.2) (layer B.Cu) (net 3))
 (segment (start 177.8 102.87) (end 154.305 102.87) (width 0.2) (layer B.Cu) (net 3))
 (segment (start 179.705 104.775) (end 177.8 102.87) (width 0.2) (layer B.Cu) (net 3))
 (segment (start 162.56 112.395) (end 161.925 112.395) (width 0.2) (layer B.Cu) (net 3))
 (segment (start 162.56 112.395) (end 162.56 114.3) (width 0.6) (layer B.Cu) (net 3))
 (segment (start 162.56 114.3) (end 163.325 115.065) (width 0.6) (layer B.Cu) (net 3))
 (segment (start 163.325 115.065) (end 167.060001 115.065) (width 0.6) (layer B.Cu) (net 3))
 (segment (start 156.21 107.315) (end 156.21 105.41) (width 0.25) (layer B.Cu) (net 5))
 (segment (start 156.21 105.41) (end 157.48 104.14) (width 0.25) (layer B.Cu) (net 5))
 (segment (start 157.48 104.14) (end 168.275 104.14) (width 0.25) (layer B.Cu) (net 5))
 (segment (start 168.275 104.14) (end 170.815 106.68) (width 0.25) (layer B.Cu) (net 5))
 (segment (start 170.815 106.68) (end 170.815 108.585) (width 0.25) (layer B.Cu) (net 5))
 (segment (start 170.815 108.585) (end 172.215 109.985) (width 0.25) (layer B.Cu) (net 5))
 (segment (start 172.215 109.985) (end 174.680001 109.985) (width 0.25) (layer B.Cu) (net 5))
 (segment (start 156.21 107.315) (end 153.035 107.315) (width 0.6) (layer B.Cu) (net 5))
 (segment (start 167.060001 112.525) (end 165.865 112.525) (width 0.2) (layer B.Cu) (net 6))
 (segment (start 183.515 111.125) (end 184.785 112.395) (width 0.2) (layer B.Cu) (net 6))
 (segment (start 171.45 111.125) (end 183.515 111.125) (width 0.2) (layer B.Cu) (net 6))
 (segment (start 168.91 108.585) (end 171.45 111.125) (width 0.2) (layer B.Cu) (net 6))
 (segment (start 166.37 108.585) (end 168.91 108.585) (width 0.2) (layer B.Cu) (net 6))
 (segment (start 165.1 109.855) (end 166.37 108.585) (width 0.2) (layer B.Cu) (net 6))
 (segment (start 165.1 111.76) (end 165.1 109.855) (width 0.2) (layer B.Cu) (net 6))
 (segment (start 165.865 112.525) (end 165.1 111.76) (width 0.2) (layer B.Cu) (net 6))
 (segment (start 159.385 112.395) (end 159.385 116.205) (width 0.6) (layer B.Cu) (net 6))
 (segment (start 169.04 112.525) (end 167.060001 112.525) (width 0.6) (layer B.Cu) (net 6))
 (segment (start 170.18 113.665) (end 169.04 112.525) (width 0.6) (layer B.Cu) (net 6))
 (segment (start 170.18 116.205) (end 170.18 113.665) (width 0.6) (layer B.Cu) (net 6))
 (segment (start 168.275 118.11) (end 170.18 116.205) (width 0.6) (layer B.Cu) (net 6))
 (segment (start 161.29 118.11) (end 168.275 118.11) (width 0.6) (layer B.Cu) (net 6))
 (segment (start 159.385 116.205) (end 161.29 118.11) (width 0.6) (layer B.Cu) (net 6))
 (segment (start 167.005 123.19) (end 167.005 124.46) (width 0.6) (layer B.Cu) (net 4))
 (segment (start 167.005 124.46) (end 167.64 125.095) (width 0.6) (layer B.Cu) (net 4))
 (segment (start 167.64 125.095) (end 186.69 125.095) (width 0.6) (layer B.Cu) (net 4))
 (segment (start 186.69 125.095) (end 187.96 123.825) (width 0.6) (layer B.Cu) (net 4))
 (segment (start 187.96 123.825) (end 187.96 107.315) (width 0.6) (layer B.Cu) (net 4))
 (segment (start 187.96 107.315) (end 187.325 106.68) (width 0.6) (layer B.Cu) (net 4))
 (segment (start 187.325 106.68) (end 184.785 106.68) (width 0.6) (layer B.Cu) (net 4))
 (segment (start 167.005 123.19) (end 154.94 123.19) (width 0.6) (layer B.Cu) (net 4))
 (segment (start 154.94 123.19) (end 153.035 121.285) (width 0.6) (layer B.Cu) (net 4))
 (segment (start 153.035 121.285) (end 153.035 112.395) (width 0.6) (layer B.Cu) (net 4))
 (segment (start 174.680001 107.445) (end 176.025 107.445) (width 0.6) (layer B.Cu) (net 4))
 (segment (start 176.025 107.445) (end 177.8 109.22) (width 0.6) (layer B.Cu) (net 4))
 (segment (start 177.8 109.22) (end 183.515 109.22) (width 0.6) (layer B.Cu) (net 4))
 (segment (start 183.515 109.22) (end 184.785 107.95) (width 0.6) (layer B.Cu) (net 4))
 (segment (start 184.785 107.95) (end 184.785 106.68) (width 0.6) (layer B.Cu) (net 4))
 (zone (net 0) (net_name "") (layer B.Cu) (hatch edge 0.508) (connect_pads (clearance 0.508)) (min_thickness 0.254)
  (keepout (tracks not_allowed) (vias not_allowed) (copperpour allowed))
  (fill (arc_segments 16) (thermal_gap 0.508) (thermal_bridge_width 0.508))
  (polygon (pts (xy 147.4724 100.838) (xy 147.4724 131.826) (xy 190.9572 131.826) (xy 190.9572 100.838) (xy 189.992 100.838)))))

